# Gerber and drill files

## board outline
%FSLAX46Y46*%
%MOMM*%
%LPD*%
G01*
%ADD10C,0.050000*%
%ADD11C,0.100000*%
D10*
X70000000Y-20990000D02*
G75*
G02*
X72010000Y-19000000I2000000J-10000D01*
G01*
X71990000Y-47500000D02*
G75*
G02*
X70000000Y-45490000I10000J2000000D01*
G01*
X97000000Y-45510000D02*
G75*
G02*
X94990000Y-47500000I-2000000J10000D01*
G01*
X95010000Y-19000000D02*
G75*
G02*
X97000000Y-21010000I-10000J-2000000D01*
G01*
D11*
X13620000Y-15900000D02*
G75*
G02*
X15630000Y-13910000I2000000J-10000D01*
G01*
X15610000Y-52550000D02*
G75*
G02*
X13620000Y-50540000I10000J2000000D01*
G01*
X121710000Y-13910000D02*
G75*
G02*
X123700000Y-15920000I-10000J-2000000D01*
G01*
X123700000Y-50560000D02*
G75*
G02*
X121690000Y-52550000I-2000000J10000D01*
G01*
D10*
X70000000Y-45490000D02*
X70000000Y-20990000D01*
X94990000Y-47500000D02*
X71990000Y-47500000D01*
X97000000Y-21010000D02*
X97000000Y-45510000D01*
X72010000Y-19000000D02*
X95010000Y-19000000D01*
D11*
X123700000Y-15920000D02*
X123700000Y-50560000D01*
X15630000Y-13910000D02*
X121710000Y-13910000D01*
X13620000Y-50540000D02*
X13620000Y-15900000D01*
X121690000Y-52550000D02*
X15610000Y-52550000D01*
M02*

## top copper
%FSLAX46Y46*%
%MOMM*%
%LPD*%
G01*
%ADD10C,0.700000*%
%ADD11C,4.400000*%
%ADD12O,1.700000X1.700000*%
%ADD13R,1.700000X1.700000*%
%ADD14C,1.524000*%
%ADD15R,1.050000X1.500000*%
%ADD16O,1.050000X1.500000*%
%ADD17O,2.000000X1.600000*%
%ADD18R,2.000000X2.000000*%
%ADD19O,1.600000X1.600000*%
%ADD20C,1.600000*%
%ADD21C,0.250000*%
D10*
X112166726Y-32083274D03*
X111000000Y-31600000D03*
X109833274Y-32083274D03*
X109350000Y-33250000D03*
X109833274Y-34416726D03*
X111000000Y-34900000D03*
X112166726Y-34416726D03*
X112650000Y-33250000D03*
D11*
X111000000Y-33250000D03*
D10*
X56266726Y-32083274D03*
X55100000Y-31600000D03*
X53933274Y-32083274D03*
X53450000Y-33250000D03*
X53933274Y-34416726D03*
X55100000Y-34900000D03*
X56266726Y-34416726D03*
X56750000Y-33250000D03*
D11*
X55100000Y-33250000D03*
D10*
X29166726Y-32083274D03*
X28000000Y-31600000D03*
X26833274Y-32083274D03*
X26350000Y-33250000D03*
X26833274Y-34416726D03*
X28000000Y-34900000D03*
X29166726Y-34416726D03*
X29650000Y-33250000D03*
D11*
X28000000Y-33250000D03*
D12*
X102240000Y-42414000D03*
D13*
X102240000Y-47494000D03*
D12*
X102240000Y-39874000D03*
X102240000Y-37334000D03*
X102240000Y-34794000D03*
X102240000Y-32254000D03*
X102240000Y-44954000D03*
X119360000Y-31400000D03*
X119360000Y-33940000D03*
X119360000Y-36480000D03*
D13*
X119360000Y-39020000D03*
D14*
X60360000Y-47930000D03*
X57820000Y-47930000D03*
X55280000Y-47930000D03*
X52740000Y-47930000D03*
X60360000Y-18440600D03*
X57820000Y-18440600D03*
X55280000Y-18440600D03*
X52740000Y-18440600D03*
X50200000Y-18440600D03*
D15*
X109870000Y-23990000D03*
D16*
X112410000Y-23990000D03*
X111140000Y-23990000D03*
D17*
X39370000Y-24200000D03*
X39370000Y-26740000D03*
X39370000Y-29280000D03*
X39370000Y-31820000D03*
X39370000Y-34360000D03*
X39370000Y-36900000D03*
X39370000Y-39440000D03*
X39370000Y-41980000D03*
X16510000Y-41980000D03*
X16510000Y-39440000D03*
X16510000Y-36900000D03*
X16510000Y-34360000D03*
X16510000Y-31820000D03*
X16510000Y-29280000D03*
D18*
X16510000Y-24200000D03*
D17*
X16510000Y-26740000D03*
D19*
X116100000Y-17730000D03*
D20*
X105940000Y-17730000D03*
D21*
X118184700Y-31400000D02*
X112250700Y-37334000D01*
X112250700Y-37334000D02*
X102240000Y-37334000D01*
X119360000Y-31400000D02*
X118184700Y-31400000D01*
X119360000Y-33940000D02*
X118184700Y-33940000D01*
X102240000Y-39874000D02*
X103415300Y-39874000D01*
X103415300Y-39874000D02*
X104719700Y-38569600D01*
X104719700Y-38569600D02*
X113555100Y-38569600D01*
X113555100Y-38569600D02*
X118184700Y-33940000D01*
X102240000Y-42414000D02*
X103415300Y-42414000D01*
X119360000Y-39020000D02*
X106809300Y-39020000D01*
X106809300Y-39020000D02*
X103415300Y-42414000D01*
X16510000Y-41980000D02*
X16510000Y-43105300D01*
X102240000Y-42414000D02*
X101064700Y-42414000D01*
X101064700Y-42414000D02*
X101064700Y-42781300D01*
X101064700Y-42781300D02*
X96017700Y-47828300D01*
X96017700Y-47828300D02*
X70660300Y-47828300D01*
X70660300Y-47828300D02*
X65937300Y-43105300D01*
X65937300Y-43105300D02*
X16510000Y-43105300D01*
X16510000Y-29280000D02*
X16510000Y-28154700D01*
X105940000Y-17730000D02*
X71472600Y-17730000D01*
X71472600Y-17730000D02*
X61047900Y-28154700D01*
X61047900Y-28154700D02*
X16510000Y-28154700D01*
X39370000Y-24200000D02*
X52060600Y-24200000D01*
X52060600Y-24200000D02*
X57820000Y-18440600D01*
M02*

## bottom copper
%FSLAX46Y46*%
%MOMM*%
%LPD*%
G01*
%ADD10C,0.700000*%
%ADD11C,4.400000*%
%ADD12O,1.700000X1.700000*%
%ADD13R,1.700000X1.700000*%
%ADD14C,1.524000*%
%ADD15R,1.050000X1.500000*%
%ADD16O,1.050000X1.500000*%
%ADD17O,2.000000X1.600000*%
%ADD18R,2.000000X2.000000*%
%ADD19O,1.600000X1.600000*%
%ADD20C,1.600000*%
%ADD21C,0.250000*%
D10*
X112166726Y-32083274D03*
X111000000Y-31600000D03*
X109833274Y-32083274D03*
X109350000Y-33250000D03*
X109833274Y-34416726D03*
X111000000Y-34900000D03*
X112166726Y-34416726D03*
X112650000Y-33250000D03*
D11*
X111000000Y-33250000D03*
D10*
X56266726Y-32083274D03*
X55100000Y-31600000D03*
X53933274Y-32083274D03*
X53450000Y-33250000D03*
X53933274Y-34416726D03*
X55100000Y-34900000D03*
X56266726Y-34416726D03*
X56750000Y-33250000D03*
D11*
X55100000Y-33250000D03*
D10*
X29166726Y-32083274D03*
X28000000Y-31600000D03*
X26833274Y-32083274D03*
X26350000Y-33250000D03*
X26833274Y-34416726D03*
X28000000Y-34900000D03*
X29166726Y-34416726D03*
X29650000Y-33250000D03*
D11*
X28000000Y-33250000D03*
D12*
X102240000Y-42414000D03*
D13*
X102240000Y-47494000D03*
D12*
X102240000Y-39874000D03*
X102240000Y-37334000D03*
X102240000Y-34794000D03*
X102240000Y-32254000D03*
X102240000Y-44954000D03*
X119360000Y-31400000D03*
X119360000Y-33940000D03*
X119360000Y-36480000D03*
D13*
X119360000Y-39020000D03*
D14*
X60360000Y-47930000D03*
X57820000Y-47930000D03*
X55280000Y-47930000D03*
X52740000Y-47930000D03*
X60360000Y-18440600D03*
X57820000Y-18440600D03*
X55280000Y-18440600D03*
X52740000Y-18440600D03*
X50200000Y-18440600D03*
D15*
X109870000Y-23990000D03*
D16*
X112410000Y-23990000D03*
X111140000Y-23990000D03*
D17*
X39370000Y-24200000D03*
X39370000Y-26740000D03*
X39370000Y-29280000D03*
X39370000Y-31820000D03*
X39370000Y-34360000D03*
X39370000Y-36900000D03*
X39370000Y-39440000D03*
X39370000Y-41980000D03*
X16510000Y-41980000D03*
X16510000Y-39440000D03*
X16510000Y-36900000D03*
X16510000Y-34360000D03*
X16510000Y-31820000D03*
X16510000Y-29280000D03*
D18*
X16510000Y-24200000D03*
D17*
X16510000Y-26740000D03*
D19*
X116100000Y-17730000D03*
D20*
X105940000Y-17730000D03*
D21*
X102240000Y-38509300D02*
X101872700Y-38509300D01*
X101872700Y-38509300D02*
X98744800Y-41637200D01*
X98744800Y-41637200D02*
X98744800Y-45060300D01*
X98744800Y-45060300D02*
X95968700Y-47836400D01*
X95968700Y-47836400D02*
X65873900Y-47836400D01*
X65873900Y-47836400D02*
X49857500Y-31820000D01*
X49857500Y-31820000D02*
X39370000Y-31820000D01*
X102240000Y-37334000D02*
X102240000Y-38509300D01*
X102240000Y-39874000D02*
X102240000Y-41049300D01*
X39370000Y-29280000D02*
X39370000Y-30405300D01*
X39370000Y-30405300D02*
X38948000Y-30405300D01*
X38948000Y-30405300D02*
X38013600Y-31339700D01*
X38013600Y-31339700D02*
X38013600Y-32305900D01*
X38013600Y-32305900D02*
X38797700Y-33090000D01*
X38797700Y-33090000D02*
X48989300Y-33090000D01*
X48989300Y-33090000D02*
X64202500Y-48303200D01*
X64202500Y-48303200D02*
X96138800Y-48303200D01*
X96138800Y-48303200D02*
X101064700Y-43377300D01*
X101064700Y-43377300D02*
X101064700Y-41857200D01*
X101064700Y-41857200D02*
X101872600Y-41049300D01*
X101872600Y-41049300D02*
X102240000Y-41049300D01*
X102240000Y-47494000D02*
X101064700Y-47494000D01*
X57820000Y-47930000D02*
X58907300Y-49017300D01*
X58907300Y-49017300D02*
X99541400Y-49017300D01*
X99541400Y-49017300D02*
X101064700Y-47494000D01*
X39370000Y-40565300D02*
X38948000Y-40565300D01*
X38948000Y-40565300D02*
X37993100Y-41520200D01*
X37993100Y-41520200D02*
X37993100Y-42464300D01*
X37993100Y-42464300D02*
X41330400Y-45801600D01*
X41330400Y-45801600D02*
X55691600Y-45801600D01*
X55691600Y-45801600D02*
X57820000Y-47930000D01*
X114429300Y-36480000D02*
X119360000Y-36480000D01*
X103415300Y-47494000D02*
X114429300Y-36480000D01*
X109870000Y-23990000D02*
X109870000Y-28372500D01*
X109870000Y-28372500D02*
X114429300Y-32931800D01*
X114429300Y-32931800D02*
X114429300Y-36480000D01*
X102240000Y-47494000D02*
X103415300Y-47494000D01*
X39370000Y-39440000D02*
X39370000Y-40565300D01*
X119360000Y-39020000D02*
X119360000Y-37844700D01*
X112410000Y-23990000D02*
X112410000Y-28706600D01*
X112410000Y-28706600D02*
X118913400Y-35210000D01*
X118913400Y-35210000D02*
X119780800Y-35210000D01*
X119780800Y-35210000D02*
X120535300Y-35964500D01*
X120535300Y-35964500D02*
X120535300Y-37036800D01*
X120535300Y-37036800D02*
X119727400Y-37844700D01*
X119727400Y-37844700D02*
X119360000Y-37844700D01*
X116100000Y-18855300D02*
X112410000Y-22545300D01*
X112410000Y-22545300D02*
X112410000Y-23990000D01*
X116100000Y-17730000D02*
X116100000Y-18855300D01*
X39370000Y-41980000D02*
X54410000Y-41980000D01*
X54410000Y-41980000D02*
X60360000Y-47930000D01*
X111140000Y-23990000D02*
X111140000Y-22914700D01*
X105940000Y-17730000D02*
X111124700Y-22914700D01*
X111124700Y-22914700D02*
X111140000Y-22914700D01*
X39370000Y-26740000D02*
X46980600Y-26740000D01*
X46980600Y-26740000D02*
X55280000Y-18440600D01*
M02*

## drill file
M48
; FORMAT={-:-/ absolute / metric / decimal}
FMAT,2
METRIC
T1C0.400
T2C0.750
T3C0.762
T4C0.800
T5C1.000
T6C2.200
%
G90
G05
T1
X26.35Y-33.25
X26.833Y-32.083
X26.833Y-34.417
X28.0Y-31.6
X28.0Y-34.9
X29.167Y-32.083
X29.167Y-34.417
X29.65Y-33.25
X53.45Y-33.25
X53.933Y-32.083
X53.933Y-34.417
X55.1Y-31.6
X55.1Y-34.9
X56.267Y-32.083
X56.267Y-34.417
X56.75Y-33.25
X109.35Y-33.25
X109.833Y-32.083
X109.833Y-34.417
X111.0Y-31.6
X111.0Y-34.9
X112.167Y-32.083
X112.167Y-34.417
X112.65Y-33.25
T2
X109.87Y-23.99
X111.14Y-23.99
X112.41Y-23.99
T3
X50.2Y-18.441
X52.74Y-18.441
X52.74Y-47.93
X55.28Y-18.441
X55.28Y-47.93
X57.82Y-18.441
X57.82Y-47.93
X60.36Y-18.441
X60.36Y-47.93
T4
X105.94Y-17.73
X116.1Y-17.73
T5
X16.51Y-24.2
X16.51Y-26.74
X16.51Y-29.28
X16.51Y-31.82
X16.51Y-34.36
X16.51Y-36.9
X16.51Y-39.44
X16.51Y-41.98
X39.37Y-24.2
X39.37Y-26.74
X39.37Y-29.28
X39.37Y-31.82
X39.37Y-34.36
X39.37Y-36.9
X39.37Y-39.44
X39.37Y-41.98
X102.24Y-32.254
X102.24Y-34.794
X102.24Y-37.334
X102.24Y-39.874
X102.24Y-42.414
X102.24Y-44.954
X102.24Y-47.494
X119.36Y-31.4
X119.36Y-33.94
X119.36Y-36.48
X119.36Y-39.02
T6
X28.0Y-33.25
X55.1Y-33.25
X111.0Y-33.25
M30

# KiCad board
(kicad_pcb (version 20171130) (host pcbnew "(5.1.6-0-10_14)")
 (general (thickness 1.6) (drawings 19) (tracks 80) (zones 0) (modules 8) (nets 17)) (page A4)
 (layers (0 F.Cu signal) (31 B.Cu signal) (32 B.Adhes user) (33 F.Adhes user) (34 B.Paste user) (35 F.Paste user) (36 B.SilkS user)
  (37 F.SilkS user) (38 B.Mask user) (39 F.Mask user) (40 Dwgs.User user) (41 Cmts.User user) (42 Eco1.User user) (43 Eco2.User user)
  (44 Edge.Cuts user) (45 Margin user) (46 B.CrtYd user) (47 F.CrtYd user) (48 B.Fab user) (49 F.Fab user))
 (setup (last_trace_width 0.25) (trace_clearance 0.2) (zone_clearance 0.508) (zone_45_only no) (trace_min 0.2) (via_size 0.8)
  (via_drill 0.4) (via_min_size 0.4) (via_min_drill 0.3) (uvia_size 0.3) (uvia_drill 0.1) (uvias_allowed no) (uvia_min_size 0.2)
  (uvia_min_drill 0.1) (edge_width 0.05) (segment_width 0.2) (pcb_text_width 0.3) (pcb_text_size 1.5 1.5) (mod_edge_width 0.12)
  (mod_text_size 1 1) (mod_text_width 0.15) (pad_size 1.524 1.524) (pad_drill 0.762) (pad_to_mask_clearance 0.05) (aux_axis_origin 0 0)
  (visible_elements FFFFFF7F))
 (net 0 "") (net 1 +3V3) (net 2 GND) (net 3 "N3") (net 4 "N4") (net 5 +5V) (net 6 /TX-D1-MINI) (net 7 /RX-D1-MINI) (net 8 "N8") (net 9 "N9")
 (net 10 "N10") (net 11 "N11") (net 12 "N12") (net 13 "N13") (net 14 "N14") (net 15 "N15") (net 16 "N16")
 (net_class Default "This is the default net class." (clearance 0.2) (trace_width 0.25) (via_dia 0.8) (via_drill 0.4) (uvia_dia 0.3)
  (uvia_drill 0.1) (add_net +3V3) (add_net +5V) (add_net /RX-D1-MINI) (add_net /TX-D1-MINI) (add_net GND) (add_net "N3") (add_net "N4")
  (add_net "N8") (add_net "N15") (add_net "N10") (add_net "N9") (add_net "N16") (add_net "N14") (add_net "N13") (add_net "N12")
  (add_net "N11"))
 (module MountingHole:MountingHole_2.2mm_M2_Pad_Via (layer F.Cu) (at 111 33.25)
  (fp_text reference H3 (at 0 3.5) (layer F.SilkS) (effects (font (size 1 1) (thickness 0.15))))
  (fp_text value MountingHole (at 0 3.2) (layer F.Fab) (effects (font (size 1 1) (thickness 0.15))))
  (pad 1 thru_hole circle (at 1.166726 -1.166726) (size 0.7 0.7) (drill 0.4) (layers *.Cu *.Mask))
  (pad 1 thru_hole circle (at 0 -1.65) (size 0.7 0.7) (drill 0.4) (layers *.Cu *.Mask))
  (pad 1 thru_hole circle (at -1.166726 -1.166726) (size 0.7 0.7) (drill 0.4) (layers *.Cu *.Mask))
  (pad 1 thru_hole circle (at -1.65 0) (size 0.7 0.7) (drill 0.4) (layers *.Cu *.Mask))
  (pad 1 thru_hole circle (at -1.166726 1.166726) (size 0.7 0.7) (drill 0.4) (layers *.Cu *.Mask))
  (pad 1 thru_hole circle (at 0 1.65) (size 0.7 0.7) (drill 0.4) (layers *.Cu *.Mask))
  (pad 1 thru_hole circle (at 1.166726 1.166726) (size 0.7 0.7) (drill 0.4) (layers *.Cu *.Mask))
  (pad 1 thru_hole circle (at 1.65 0) (size 0.7 0.7) (drill 0.4) (layers *.Cu *.Mask))
  (pad 1 thru_hole circle (at 0 0) (size 4.4 4.4) (drill 2.2) (layers *.Cu *.Mask)))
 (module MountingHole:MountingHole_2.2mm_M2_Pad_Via (layer F.Cu) (at 55.1 33.25)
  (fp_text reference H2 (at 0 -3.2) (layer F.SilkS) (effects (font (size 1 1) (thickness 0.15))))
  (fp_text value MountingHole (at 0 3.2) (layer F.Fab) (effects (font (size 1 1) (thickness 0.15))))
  (pad 1 thru_hole circle (at 1.166726 -1.166726) (size 0.7 0.7) (drill 0.4) (layers *.Cu *.Mask))
  (pad 1 thru_hole circle (at 0 -1.65) (size 0.7 0.7) (drill 0.4) (layers *.Cu *.Mask))
  (pad 1 thru_hole circle (at -1.166726 -1.166726) (size 0.7 0.7) (drill 0.4) (layers *.Cu *.Mask))
  (pad 1 thru_hole circle (at -1.65 0) (size 0.7 0.7) (drill 0.4) (layers *.Cu *.Mask))
  (pad 1 thru_hole circle (at -1.166726 1.166726) (size 0.7 0.7) (drill 0.4) (layers *.Cu *.Mask))
  (pad 1 thru_hole circle (at 0 1.65) (size 0.7 0.7) (drill 0.4) (layers *.Cu *.Mask))
  (pad 1 thru_hole circle (at 1.166726 1.166726) (size 0.7 0.7) (drill 0.4) (layers *.Cu *.Mask))
  (pad 1 thru_hole circle (at 1.65 0) (size 0.7 0.7) (drill 0.4) (layers *.Cu *.Mask))
  (pad 1 thru_hole circle (at 0 0) (size 4.4 4.4) (drill 2.2) (layers *.Cu *.Mask)))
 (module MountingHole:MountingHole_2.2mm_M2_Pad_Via (layer F.Cu) (at 28 33.25)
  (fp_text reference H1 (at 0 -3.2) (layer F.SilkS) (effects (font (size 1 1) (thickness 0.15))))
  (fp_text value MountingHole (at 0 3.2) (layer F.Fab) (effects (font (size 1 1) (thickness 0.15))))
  (pad 1 thru_hole circle (at 1.166726 -1.166726) (size 0.7 0.7) (drill 0.4) (layers *.Cu *.Mask))
  (pad 1 thru_hole circle (at 0 -1.65) (size 0.7 0.7) (drill 0.4) (layers *.Cu *.Mask))
  (pad 1 thru_hole circle (at -1.166726 -1.166726) (size 0.7 0.7) (drill 0.4) (layers *.Cu *.Mask))
  (pad 1 thru_hole circle (at -1.65 0) (size 0.7 0.7) (drill 0.4) (layers *.Cu *.Mask))
  (pad 1 thru_hole circle (at -1.166726 1.166726) (size 0.7 0.7) (drill 0.4) (layers *.Cu *.Mask))
  (pad 1 thru_hole circle (at 0 1.65) (size 0.7 0.7) (drill 0.4) (layers *.Cu *.Mask))
  (pad 1 thru_hole circle (at 1.166726 1.166726) (size 0.7 0.7) (drill 0.4) (layers *.Cu *.Mask))
  (pad 1 thru_hole circle (at 1.65 0) (size 0.7 0.7) (drill 0.4) (layers *.Cu *.Mask))
  (pad 1 thru_hole circle (at 0 0) (size 4.4 4.4) (drill 2.2) (layers *.Cu *.Mask)))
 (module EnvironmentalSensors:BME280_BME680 (layer F.Cu) (at 119.36 39.02 180)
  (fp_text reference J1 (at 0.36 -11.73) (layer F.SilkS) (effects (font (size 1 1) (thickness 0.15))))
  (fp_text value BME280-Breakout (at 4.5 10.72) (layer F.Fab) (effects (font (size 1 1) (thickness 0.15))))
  (pad 1 thru_hole oval (at 17.12 -3.394 180) (size 1.7 1.7) (drill 1) (layers *.Cu *.Mask) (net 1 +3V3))
  (pad 2 thru_hole rect (at 17.12 -8.474 180) (size 1.7 1.7) (drill 1) (layers *.Cu *.Mask) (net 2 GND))
  (pad 3 thru_hole oval (at 17.12 -0.854 180) (size 1.7 1.7) (drill 1) (layers *.Cu *.Mask) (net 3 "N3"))
  (pad 4 thru_hole oval (at 17.12 1.686 180) (size 1.7 1.7) (drill 1) (layers *.Cu *.Mask) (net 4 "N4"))
  (pad "" thru_hole oval (at 17.12 4.226 180) (size 1.7 1.7) (drill 1) (layers *.Cu *.Mask))
  (pad "" thru_hole oval (at 17.12 6.766 180) (size 1.7 1.7) (drill 1) (layers *.Cu *.Mask))
  (pad "" thru_hole oval (at 17.12 -5.934 180) (size 1.7 1.7) (drill 1) (layers *.Cu *.Mask))
  (pad 4 thru_hole oval (at 0 7.62 180) (size 1.7 1.7) (drill 1) (layers *.Cu *.Mask) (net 4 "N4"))
  (pad 3 thru_hole oval (at 0 5.08 180) (size 1.7 1.7) (drill 1) (layers *.Cu *.Mask) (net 3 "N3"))
  (pad 2 thru_hole oval (at 0 2.54 180) (size 1.7 1.7) (drill 1) (layers *.Cu *.Mask) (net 2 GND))
  (pad 1 thru_hole rect (at 0 0 180) (size 1.7 1.7) (drill 1) (layers *.Cu *.Mask) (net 1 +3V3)))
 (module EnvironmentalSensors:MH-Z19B (layer F.Cu) (at 60.36 47.93 90)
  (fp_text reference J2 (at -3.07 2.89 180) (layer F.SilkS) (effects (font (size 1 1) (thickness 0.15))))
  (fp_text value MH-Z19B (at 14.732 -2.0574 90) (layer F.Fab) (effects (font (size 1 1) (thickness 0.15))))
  (pad 1 thru_hole circle (at 0 0 90) (size 1.524 1.524) (drill 0.762) (layers *.Cu *.Mask) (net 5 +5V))
  (pad 2 thru_hole circle (at 0 -2.54 90) (size 1.524 1.524) (drill 0.762) (layers *.Cu *.Mask) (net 2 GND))
  (pad 3 thru_hole circle (at 0 -5.08 90) (size 1.524 1.524) (drill 0.762) (layers *.Cu *.Mask))
  (pad 4 thru_hole circle (at 0 -7.62 90) (size 1.524 1.524) (drill 0.762) (layers *.Cu *.Mask))
  (pad 5 thru_hole circle (at 29.4894 0 90) (size 1.524 1.524) (drill 0.762) (layers *.Cu *.Mask))
  (pad 6 thru_hole circle (at 29.4894 -2.54 90) (size 1.524 1.524) (drill 0.762) (layers *.Cu *.Mask) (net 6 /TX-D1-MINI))
  (pad 7 thru_hole circle (at 29.4894 -5.08 90) (size 1.524 1.524) (drill 0.762) (layers *.Cu *.Mask) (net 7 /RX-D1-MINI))
  (pad 8 thru_hole circle (at 29.4894 -7.62 90) (size 1.524 1.524) (drill 0.762) (layers *.Cu *.Mask))
  (pad 9 thru_hole circle (at 29.4894 -10.16 90) (size 1.524 1.524) (drill 0.762) (layers *.Cu *.Mask)))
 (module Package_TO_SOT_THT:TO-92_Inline (layer F.Cu) (at 109.87 23.99)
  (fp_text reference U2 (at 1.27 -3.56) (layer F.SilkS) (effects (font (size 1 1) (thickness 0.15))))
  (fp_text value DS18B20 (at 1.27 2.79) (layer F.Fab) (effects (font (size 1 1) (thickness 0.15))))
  (pad 1 thru_hole rect (at 0 0) (size 1.05 1.5) (drill 0.75) (layers *.Cu *.Mask) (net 2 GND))
  (pad 3 thru_hole oval (at 2.54 0) (size 1.05 1.5) (drill 0.75) (layers *.Cu *.Mask) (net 1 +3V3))
  (pad 2 thru_hole oval (at 1.27 0) (size 1.05 1.5) (drill 0.75) (layers *.Cu *.Mask) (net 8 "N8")))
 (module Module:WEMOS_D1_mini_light (layer F.Cu) (at 16.51 24.2)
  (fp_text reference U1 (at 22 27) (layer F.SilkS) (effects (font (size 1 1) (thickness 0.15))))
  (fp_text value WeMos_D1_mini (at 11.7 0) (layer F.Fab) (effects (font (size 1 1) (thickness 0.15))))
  (pad 16 thru_hole oval (at 22.86 0) (size 2 1.6) (drill 1) (layers *.Cu *.Mask) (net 6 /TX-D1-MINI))
  (pad 15 thru_hole oval (at 22.86 2.54) (size 2 1.6) (drill 1) (layers *.Cu *.Mask) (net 7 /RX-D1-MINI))
  (pad 14 thru_hole oval (at 22.86 5.08) (size 2 1.6) (drill 1) (layers *.Cu *.Mask) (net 3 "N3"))
  (pad 13 thru_hole oval (at 22.86 7.62) (size 2 1.6) (drill 1) (layers *.Cu *.Mask) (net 4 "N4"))
  (pad 12 thru_hole oval (at 22.86 10.16) (size 2 1.6) (drill 1) (layers *.Cu *.Mask) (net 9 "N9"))
  (pad 11 thru_hole oval (at 22.86 12.7) (size 2 1.6) (drill 1) (layers *.Cu *.Mask) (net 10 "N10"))
  (pad 10 thru_hole oval (at 22.86 15.24) (size 2 1.6) (drill 1) (layers *.Cu *.Mask) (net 2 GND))
  (pad 9 thru_hole oval (at 22.86 17.78) (size 2 1.6) (drill 1) (layers *.Cu *.Mask) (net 5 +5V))
  (pad 8 thru_hole oval (at 0 17.78) (size 2 1.6) (drill 1) (layers *.Cu *.Mask) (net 1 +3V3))
  (pad 7 thru_hole oval (at 0 15.24) (size 2 1.6) (drill 1) (layers *.Cu *.Mask) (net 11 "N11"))
  (pad 6 thru_hole oval (at 0 12.7) (size 2 1.6) (drill 1) (layers *.Cu *.Mask) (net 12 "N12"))
  (pad 5 thru_hole oval (at 0 10.16) (size 2 1.6) (drill 1) (layers *.Cu *.Mask) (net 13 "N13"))
  (pad 4 thru_hole oval (at 0 7.62) (size 2 1.6) (drill 1) (layers *.Cu *.Mask) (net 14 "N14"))
  (pad 3 thru_hole oval (at 0 5.08) (size 2 1.6) (drill 1) (layers *.Cu *.Mask) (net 8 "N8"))
  (pad 1 thru_hole rect (at 0 0) (size 2 2) (drill 1) (layers *.Cu *.Mask) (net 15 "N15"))
  (pad 2 thru_hole oval (at 0 2.54) (size 2 1.6) (drill 1) (layers *.Cu *.Mask) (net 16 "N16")))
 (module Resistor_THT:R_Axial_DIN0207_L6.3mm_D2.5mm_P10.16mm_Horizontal (layer F.Cu) (at 105.94 17.73)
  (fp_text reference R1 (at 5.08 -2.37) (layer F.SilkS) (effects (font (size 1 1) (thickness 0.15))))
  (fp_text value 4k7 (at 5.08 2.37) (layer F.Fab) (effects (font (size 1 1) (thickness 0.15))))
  (pad 2 thru_hole oval (at 10.16 0) (size 1.6 1.6) (drill 0.8) (layers *.Cu *.Mask) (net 1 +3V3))
  (pad 1 thru_hole circle (at 0 0) (size 1.6 1.6) (drill 0.8) (layers *.Cu *.Mask) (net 8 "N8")))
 (gr_arc (start 72 21) (end 72.01 19) (angle -90) (layer Edge.Cuts) (width 0.05))
 (gr_arc (start 72 45.5) (end 70 45.49) (angle -90) (layer Edge.Cuts) (width 0.05))
 (gr_arc (start 95 45.5) (end 94.99 47.5) (angle -90) (layer Edge.Cuts) (width 0.05))
 (gr_arc (start 95 21) (end 97 21.01) (angle -90) (layer Edge.Cuts) (width 0.05))
 (gr_arc (start 15.62 15.91) (end 15.63 13.91) (angle -90) (layer Edge.Cuts) (width 0.1))
 (gr_arc (start 15.62 50.55) (end 13.62 50.54) (angle -90) (layer Edge.Cuts) (width 0.1))
 (gr_arc (start 121.7 15.91) (end 123.7 15.92) (angle -90) (layer Edge.Cuts) (width 0.1))
 (gr_arc (start 121.7 50.55) (end 121.69 52.55) (angle -90) (layer Edge.Cuts) (width 0.1))
 (gr_line (start 70 45.49) (end 70 20.99) (layer Edge.Cuts) (width 0.05))
 (gr_line (start 94.99 47.5) (end 71.99 47.5) (layer Edge.Cuts) (width 0.05))
 (gr_line (start 97 21.01) (end 97 45.51) (layer Edge.Cuts) (width 0.05))
 (gr_line (start 72.01 19) (end 95.01 19) (layer Edge.Cuts) (width 0.05))
 (gr_line (start 123.7 15.92) (end 123.7 50.56) (layer Edge.Cuts) (width 0.1))
 (gr_line (start 15.63 13.91) (end 121.71 13.91) (layer Edge.Cuts) (width 0.1))
 (gr_line (start 13.62 50.54) (end 13.62 15.9) (layer Edge.Cuts) (width 0.1))
 (gr_line (start 121.69 52.55) (end 15.61 52.55) (layer Edge.Cuts) (width 0.1))
 (segment (start 118.1847 31.4) (end 112.2507 37.334) (width 0.25) (layer F.Cu) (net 4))
 (segment (start 112.2507 37.334) (end 102.24 37.334) (width 0.25) (layer F.Cu) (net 4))
 (segment (start 102.24 38.5093) (end 101.8727 38.5093) (width 0.25) (layer B.Cu) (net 4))
 (segment (start 101.8727 38.5093) (end 98.7448 41.6372) (width 0.25) (layer B.Cu) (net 4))
 (segment (start 98.7448 41.6372) (end 98.7448 45.0603) (width 0.25) (layer B.Cu) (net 4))
 (segment (start 98.7448 45.0603) (end 95.9687 47.8364) (width 0.25) (layer B.Cu) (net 4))
 (segment (start 95.9687 47.8364) (end 65.8739 47.8364) (width 0.25) (layer B.Cu) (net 4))
 (segment (start 65.8739 47.8364) (end 49.8575 31.82) (width 0.25) (layer B.Cu) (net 4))
 (segment (start 49.8575 31.82) (end 39.37 31.82) (width 0.25) (layer B.Cu) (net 4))
 (segment (start 102.24 37.334) (end 102.24 38.5093) (width 0.25) (layer B.Cu) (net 4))
 (segment (start 119.36 31.4) (end 118.1847 31.4) (width 0.25) (layer F.Cu) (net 4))
 (segment (start 119.36 33.94) (end 118.1847 33.94) (width 0.25) (layer F.Cu) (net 3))
 (segment (start 102.24 39.874) (end 103.4153 39.874) (width 0.25) (layer F.Cu) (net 3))
 (segment (start 103.4153 39.874) (end 104.7197 38.5696) (width 0.25) (layer F.Cu) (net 3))
 (segment (start 104.7197 38.5696) (end 113.5551 38.5696) (width 0.25) (layer F.Cu) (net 3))
 (segment (start 113.5551 38.5696) (end 118.1847 33.94) (width 0.25) (layer F.Cu) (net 3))
 (segment (start 102.24 39.874) (end 102.24 41.0493) (width 0.25) (layer B.Cu) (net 3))
 (segment (start 39.37 29.28) (end 39.37 30.4053) (width 0.25) (layer B.Cu) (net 3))
 (segment (start 39.37 30.4053) (end 38.948 30.4053) (width 0.25) (layer B.Cu) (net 3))
 (segment (start 38.948 30.4053) (end 38.0136 31.3397) (width 0.25) (layer B.Cu) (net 3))
 (segment (start 38.0136 31.3397) (end 38.0136 32.3059) (width 0.25) (layer B.Cu) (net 3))
 (segment (start 38.0136 32.3059) (end 38.7977 33.09) (width 0.25) (layer B.Cu) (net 3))
 (segment (start 38.7977 33.09) (end 48.9893 33.09) (width 0.25) (layer B.Cu) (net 3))
 (segment (start 48.9893 33.09) (end 64.2025 48.3032) (width 0.25) (layer B.Cu) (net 3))
 (segment (start 64.2025 48.3032) (end 96.1388 48.3032) (width 0.25) (layer B.Cu) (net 3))
 (segment (start 96.1388 48.3032) (end 101.0647 43.3773) (width 0.25) (layer B.Cu) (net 3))
 (segment (start 101.0647 43.3773) (end 101.0647 41.8572) (width 0.25) (layer B.Cu) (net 3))
 (segment (start 101.0647 41.8572) (end 101.8726 41.0493) (width 0.25) (layer B.Cu) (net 3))
 (segment (start 101.8726 41.0493) (end 102.24 41.0493) (width 0.25) (layer B.Cu) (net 3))
 (segment (start 102.24 47.494) (end 101.0647 47.494) (width 0.25) (layer B.Cu) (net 2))
 (segment (start 57.82 47.93) (end 58.9073 49.0173) (width 0.25) (layer B.Cu) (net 2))
 (segment (start 58.9073 49.0173) (end 99.5414 49.0173) (width 0.25) (layer B.Cu) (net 2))
 (segment (start 99.5414 49.0173) (end 101.0647 47.494) (width 0.25) (layer B.Cu) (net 2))
 (segment (start 39.37 40.5653) (end 38.948 40.5653) (width 0.25) (layer B.Cu) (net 2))
 (segment (start 38.948 40.5653) (end 37.9931 41.5202) (width 0.25) (layer B.Cu) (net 2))
 (segment (start 37.9931 41.5202) (end 37.9931 42.4643) (width 0.25) (layer B.Cu) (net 2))
 (segment (start 37.9931 42.4643) (end 41.3304 45.8016) (width 0.25) (layer B.Cu) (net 2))
 (segment (start 41.3304 45.8016) (end 55.6916 45.8016) (width 0.25) (layer B.Cu) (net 2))
 (segment (start 55.6916 45.8016) (end 57.82 47.93) (width 0.25) (layer B.Cu) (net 2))
 (segment (start 114.4293 36.48) (end 119.36 36.48) (width 0.25) (layer B.Cu) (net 2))
 (segment (start 103.4153 47.494) (end 114.4293 36.48) (width 0.25) (layer B.Cu) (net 2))
 (segment (start 109.87 23.99) (end 109.87 28.3725) (width 0.25) (layer B.Cu) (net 2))
 (segment (start 109.87 28.3725) (end 114.4293 32.9318) (width 0.25) (layer B.Cu) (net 2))
 (segment (start 114.4293 32.9318) (end 114.4293 36.48) (width 0.25) (layer B.Cu) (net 2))
 (segment (start 102.24 47.494) (end 103.4153 47.494) (width 0.25) (layer B.Cu) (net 2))
 (segment (start 39.37 39.44) (end 39.37 40.5653) (width 0.25) (layer B.Cu) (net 2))
 (segment (start 119.36 39.02) (end 119.36 37.8447) (width 0.25) (layer B.Cu) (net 1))
 (segment (start 112.41 23.99) (end 112.41 28.7066) (width 0.25) (layer B.Cu) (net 1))
 (segment (start 112.41 28.7066) (end 118.9134 35.21) (width 0.25) (layer B.Cu) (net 1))
 (segment (start 118.9134 35.21) (end 119.7808 35.21) (width 0.25) (layer B.Cu) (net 1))
 (segment (start 119.7808 35.21) (end 120.5353 35.9645) (width 0.25) (layer B.Cu) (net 1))
 (segment (start 120.5353 35.9645) (end 120.5353 37.0368) (width 0.25) (layer B.Cu) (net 1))
 (segment (start 120.5353 37.0368) (end 119.7274 37.8447) (width 0.25) (layer B.Cu) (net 1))
 (segment (start 119.7274 37.8447) (end 119.36 37.8447) (width 0.25) (layer B.Cu) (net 1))
 (segment (start 116.1 18.8553) (end 112.41 22.5453) (width 0.25) (layer B.Cu) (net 1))
 (segment (start 112.41 22.5453) (end 112.41 23.99) (width 0.25) (layer B.Cu) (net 1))
 (segment (start 116.1 17.73) (end 116.1 18.8553) (width 0.25) (layer B.Cu) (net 1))
 (segment (start 102.24 42.414) (end 103.4153 42.414) (width 0.25) (layer F.Cu) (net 1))
 (segment (start 119.36 39.02) (end 106.8093 39.02) (width 0.25) (layer F.Cu) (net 1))
 (segment (start 106.8093 39.02) (end 103.4153 42.414) (width 0.25) (layer F.Cu) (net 1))
 (segment (start 16.51 41.98) (end 16.51 43.1053) (width 0.25) (layer F.Cu) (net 1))
 (segment (start 102.24 42.414) (end 101.0647 42.414) (width 0.25) (layer F.Cu) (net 1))
 (segment (start 101.0647 42.414) (end 101.0647 42.7813) (width 0.25) (layer F.Cu) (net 1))
 (segment (start 101.0647 42.7813) (end 96.0177 47.8283) (width 0.25) (layer F.Cu) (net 1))
 (segment (start 96.0177 47.8283) (end 70.6603 47.8283) (width 0.25) (layer F.Cu) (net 1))
 (segment (start 70.6603 47.8283) (end 65.9373 43.1053) (width 0.25) (layer F.Cu) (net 1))
 (segment (start 65.9373 43.1053) (end 16.51 43.1053) (width 0.25) (layer F.Cu) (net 1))
 (segment (start 39.37 41.98) (end 54.41 41.98) (width 0.25) (layer B.Cu) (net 5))
 (segment (start 54.41 41.98) (end 60.36 47.93) (width 0.25) (layer B.Cu) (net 5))
 (segment (start 16.51 29.28) (end 16.51 28.1547) (width 0.25) (layer F.Cu) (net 8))
 (segment (start 105.94 17.73) (end 71.4726 17.73) (width 0.25) (layer F.Cu) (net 8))
 (segment (start 71.4726 17.73) (end 61.0479 28.1547) (width 0.25) (layer F.Cu) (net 8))
 (segment (start 61.0479 28.1547) (end 16.51 28.1547) (width 0.25) (layer F.Cu) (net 8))
 (segment (start 111.14 23.99) (end 111.14 22.9147) (width 0.25) (layer B.Cu) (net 8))
 (segment (start 105.94 17.73) (end 111.1247 22.9147) (width 0.25) (layer B.Cu) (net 8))
 (segment (start 111.1247 22.9147) (end 111.14 22.9147) (width 0.25) (layer B.Cu) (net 8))
 (segment (start 39.37 24.2) (end 52.0606 24.2) (width 0.25) (layer F.Cu) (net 6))
 (segment (start 52.0606 24.2) (end 57.82 18.4406) (width 0.25) (layer F.Cu) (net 6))
 (segment (start 39.37 26.74) (end 46.9806 26.74) (width 0.25) (layer B.Cu) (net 7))
 (segment (start 46.9806 26.74) (end 55.28 18.4406) (width 0.25) (layer B.Cu) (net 7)))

